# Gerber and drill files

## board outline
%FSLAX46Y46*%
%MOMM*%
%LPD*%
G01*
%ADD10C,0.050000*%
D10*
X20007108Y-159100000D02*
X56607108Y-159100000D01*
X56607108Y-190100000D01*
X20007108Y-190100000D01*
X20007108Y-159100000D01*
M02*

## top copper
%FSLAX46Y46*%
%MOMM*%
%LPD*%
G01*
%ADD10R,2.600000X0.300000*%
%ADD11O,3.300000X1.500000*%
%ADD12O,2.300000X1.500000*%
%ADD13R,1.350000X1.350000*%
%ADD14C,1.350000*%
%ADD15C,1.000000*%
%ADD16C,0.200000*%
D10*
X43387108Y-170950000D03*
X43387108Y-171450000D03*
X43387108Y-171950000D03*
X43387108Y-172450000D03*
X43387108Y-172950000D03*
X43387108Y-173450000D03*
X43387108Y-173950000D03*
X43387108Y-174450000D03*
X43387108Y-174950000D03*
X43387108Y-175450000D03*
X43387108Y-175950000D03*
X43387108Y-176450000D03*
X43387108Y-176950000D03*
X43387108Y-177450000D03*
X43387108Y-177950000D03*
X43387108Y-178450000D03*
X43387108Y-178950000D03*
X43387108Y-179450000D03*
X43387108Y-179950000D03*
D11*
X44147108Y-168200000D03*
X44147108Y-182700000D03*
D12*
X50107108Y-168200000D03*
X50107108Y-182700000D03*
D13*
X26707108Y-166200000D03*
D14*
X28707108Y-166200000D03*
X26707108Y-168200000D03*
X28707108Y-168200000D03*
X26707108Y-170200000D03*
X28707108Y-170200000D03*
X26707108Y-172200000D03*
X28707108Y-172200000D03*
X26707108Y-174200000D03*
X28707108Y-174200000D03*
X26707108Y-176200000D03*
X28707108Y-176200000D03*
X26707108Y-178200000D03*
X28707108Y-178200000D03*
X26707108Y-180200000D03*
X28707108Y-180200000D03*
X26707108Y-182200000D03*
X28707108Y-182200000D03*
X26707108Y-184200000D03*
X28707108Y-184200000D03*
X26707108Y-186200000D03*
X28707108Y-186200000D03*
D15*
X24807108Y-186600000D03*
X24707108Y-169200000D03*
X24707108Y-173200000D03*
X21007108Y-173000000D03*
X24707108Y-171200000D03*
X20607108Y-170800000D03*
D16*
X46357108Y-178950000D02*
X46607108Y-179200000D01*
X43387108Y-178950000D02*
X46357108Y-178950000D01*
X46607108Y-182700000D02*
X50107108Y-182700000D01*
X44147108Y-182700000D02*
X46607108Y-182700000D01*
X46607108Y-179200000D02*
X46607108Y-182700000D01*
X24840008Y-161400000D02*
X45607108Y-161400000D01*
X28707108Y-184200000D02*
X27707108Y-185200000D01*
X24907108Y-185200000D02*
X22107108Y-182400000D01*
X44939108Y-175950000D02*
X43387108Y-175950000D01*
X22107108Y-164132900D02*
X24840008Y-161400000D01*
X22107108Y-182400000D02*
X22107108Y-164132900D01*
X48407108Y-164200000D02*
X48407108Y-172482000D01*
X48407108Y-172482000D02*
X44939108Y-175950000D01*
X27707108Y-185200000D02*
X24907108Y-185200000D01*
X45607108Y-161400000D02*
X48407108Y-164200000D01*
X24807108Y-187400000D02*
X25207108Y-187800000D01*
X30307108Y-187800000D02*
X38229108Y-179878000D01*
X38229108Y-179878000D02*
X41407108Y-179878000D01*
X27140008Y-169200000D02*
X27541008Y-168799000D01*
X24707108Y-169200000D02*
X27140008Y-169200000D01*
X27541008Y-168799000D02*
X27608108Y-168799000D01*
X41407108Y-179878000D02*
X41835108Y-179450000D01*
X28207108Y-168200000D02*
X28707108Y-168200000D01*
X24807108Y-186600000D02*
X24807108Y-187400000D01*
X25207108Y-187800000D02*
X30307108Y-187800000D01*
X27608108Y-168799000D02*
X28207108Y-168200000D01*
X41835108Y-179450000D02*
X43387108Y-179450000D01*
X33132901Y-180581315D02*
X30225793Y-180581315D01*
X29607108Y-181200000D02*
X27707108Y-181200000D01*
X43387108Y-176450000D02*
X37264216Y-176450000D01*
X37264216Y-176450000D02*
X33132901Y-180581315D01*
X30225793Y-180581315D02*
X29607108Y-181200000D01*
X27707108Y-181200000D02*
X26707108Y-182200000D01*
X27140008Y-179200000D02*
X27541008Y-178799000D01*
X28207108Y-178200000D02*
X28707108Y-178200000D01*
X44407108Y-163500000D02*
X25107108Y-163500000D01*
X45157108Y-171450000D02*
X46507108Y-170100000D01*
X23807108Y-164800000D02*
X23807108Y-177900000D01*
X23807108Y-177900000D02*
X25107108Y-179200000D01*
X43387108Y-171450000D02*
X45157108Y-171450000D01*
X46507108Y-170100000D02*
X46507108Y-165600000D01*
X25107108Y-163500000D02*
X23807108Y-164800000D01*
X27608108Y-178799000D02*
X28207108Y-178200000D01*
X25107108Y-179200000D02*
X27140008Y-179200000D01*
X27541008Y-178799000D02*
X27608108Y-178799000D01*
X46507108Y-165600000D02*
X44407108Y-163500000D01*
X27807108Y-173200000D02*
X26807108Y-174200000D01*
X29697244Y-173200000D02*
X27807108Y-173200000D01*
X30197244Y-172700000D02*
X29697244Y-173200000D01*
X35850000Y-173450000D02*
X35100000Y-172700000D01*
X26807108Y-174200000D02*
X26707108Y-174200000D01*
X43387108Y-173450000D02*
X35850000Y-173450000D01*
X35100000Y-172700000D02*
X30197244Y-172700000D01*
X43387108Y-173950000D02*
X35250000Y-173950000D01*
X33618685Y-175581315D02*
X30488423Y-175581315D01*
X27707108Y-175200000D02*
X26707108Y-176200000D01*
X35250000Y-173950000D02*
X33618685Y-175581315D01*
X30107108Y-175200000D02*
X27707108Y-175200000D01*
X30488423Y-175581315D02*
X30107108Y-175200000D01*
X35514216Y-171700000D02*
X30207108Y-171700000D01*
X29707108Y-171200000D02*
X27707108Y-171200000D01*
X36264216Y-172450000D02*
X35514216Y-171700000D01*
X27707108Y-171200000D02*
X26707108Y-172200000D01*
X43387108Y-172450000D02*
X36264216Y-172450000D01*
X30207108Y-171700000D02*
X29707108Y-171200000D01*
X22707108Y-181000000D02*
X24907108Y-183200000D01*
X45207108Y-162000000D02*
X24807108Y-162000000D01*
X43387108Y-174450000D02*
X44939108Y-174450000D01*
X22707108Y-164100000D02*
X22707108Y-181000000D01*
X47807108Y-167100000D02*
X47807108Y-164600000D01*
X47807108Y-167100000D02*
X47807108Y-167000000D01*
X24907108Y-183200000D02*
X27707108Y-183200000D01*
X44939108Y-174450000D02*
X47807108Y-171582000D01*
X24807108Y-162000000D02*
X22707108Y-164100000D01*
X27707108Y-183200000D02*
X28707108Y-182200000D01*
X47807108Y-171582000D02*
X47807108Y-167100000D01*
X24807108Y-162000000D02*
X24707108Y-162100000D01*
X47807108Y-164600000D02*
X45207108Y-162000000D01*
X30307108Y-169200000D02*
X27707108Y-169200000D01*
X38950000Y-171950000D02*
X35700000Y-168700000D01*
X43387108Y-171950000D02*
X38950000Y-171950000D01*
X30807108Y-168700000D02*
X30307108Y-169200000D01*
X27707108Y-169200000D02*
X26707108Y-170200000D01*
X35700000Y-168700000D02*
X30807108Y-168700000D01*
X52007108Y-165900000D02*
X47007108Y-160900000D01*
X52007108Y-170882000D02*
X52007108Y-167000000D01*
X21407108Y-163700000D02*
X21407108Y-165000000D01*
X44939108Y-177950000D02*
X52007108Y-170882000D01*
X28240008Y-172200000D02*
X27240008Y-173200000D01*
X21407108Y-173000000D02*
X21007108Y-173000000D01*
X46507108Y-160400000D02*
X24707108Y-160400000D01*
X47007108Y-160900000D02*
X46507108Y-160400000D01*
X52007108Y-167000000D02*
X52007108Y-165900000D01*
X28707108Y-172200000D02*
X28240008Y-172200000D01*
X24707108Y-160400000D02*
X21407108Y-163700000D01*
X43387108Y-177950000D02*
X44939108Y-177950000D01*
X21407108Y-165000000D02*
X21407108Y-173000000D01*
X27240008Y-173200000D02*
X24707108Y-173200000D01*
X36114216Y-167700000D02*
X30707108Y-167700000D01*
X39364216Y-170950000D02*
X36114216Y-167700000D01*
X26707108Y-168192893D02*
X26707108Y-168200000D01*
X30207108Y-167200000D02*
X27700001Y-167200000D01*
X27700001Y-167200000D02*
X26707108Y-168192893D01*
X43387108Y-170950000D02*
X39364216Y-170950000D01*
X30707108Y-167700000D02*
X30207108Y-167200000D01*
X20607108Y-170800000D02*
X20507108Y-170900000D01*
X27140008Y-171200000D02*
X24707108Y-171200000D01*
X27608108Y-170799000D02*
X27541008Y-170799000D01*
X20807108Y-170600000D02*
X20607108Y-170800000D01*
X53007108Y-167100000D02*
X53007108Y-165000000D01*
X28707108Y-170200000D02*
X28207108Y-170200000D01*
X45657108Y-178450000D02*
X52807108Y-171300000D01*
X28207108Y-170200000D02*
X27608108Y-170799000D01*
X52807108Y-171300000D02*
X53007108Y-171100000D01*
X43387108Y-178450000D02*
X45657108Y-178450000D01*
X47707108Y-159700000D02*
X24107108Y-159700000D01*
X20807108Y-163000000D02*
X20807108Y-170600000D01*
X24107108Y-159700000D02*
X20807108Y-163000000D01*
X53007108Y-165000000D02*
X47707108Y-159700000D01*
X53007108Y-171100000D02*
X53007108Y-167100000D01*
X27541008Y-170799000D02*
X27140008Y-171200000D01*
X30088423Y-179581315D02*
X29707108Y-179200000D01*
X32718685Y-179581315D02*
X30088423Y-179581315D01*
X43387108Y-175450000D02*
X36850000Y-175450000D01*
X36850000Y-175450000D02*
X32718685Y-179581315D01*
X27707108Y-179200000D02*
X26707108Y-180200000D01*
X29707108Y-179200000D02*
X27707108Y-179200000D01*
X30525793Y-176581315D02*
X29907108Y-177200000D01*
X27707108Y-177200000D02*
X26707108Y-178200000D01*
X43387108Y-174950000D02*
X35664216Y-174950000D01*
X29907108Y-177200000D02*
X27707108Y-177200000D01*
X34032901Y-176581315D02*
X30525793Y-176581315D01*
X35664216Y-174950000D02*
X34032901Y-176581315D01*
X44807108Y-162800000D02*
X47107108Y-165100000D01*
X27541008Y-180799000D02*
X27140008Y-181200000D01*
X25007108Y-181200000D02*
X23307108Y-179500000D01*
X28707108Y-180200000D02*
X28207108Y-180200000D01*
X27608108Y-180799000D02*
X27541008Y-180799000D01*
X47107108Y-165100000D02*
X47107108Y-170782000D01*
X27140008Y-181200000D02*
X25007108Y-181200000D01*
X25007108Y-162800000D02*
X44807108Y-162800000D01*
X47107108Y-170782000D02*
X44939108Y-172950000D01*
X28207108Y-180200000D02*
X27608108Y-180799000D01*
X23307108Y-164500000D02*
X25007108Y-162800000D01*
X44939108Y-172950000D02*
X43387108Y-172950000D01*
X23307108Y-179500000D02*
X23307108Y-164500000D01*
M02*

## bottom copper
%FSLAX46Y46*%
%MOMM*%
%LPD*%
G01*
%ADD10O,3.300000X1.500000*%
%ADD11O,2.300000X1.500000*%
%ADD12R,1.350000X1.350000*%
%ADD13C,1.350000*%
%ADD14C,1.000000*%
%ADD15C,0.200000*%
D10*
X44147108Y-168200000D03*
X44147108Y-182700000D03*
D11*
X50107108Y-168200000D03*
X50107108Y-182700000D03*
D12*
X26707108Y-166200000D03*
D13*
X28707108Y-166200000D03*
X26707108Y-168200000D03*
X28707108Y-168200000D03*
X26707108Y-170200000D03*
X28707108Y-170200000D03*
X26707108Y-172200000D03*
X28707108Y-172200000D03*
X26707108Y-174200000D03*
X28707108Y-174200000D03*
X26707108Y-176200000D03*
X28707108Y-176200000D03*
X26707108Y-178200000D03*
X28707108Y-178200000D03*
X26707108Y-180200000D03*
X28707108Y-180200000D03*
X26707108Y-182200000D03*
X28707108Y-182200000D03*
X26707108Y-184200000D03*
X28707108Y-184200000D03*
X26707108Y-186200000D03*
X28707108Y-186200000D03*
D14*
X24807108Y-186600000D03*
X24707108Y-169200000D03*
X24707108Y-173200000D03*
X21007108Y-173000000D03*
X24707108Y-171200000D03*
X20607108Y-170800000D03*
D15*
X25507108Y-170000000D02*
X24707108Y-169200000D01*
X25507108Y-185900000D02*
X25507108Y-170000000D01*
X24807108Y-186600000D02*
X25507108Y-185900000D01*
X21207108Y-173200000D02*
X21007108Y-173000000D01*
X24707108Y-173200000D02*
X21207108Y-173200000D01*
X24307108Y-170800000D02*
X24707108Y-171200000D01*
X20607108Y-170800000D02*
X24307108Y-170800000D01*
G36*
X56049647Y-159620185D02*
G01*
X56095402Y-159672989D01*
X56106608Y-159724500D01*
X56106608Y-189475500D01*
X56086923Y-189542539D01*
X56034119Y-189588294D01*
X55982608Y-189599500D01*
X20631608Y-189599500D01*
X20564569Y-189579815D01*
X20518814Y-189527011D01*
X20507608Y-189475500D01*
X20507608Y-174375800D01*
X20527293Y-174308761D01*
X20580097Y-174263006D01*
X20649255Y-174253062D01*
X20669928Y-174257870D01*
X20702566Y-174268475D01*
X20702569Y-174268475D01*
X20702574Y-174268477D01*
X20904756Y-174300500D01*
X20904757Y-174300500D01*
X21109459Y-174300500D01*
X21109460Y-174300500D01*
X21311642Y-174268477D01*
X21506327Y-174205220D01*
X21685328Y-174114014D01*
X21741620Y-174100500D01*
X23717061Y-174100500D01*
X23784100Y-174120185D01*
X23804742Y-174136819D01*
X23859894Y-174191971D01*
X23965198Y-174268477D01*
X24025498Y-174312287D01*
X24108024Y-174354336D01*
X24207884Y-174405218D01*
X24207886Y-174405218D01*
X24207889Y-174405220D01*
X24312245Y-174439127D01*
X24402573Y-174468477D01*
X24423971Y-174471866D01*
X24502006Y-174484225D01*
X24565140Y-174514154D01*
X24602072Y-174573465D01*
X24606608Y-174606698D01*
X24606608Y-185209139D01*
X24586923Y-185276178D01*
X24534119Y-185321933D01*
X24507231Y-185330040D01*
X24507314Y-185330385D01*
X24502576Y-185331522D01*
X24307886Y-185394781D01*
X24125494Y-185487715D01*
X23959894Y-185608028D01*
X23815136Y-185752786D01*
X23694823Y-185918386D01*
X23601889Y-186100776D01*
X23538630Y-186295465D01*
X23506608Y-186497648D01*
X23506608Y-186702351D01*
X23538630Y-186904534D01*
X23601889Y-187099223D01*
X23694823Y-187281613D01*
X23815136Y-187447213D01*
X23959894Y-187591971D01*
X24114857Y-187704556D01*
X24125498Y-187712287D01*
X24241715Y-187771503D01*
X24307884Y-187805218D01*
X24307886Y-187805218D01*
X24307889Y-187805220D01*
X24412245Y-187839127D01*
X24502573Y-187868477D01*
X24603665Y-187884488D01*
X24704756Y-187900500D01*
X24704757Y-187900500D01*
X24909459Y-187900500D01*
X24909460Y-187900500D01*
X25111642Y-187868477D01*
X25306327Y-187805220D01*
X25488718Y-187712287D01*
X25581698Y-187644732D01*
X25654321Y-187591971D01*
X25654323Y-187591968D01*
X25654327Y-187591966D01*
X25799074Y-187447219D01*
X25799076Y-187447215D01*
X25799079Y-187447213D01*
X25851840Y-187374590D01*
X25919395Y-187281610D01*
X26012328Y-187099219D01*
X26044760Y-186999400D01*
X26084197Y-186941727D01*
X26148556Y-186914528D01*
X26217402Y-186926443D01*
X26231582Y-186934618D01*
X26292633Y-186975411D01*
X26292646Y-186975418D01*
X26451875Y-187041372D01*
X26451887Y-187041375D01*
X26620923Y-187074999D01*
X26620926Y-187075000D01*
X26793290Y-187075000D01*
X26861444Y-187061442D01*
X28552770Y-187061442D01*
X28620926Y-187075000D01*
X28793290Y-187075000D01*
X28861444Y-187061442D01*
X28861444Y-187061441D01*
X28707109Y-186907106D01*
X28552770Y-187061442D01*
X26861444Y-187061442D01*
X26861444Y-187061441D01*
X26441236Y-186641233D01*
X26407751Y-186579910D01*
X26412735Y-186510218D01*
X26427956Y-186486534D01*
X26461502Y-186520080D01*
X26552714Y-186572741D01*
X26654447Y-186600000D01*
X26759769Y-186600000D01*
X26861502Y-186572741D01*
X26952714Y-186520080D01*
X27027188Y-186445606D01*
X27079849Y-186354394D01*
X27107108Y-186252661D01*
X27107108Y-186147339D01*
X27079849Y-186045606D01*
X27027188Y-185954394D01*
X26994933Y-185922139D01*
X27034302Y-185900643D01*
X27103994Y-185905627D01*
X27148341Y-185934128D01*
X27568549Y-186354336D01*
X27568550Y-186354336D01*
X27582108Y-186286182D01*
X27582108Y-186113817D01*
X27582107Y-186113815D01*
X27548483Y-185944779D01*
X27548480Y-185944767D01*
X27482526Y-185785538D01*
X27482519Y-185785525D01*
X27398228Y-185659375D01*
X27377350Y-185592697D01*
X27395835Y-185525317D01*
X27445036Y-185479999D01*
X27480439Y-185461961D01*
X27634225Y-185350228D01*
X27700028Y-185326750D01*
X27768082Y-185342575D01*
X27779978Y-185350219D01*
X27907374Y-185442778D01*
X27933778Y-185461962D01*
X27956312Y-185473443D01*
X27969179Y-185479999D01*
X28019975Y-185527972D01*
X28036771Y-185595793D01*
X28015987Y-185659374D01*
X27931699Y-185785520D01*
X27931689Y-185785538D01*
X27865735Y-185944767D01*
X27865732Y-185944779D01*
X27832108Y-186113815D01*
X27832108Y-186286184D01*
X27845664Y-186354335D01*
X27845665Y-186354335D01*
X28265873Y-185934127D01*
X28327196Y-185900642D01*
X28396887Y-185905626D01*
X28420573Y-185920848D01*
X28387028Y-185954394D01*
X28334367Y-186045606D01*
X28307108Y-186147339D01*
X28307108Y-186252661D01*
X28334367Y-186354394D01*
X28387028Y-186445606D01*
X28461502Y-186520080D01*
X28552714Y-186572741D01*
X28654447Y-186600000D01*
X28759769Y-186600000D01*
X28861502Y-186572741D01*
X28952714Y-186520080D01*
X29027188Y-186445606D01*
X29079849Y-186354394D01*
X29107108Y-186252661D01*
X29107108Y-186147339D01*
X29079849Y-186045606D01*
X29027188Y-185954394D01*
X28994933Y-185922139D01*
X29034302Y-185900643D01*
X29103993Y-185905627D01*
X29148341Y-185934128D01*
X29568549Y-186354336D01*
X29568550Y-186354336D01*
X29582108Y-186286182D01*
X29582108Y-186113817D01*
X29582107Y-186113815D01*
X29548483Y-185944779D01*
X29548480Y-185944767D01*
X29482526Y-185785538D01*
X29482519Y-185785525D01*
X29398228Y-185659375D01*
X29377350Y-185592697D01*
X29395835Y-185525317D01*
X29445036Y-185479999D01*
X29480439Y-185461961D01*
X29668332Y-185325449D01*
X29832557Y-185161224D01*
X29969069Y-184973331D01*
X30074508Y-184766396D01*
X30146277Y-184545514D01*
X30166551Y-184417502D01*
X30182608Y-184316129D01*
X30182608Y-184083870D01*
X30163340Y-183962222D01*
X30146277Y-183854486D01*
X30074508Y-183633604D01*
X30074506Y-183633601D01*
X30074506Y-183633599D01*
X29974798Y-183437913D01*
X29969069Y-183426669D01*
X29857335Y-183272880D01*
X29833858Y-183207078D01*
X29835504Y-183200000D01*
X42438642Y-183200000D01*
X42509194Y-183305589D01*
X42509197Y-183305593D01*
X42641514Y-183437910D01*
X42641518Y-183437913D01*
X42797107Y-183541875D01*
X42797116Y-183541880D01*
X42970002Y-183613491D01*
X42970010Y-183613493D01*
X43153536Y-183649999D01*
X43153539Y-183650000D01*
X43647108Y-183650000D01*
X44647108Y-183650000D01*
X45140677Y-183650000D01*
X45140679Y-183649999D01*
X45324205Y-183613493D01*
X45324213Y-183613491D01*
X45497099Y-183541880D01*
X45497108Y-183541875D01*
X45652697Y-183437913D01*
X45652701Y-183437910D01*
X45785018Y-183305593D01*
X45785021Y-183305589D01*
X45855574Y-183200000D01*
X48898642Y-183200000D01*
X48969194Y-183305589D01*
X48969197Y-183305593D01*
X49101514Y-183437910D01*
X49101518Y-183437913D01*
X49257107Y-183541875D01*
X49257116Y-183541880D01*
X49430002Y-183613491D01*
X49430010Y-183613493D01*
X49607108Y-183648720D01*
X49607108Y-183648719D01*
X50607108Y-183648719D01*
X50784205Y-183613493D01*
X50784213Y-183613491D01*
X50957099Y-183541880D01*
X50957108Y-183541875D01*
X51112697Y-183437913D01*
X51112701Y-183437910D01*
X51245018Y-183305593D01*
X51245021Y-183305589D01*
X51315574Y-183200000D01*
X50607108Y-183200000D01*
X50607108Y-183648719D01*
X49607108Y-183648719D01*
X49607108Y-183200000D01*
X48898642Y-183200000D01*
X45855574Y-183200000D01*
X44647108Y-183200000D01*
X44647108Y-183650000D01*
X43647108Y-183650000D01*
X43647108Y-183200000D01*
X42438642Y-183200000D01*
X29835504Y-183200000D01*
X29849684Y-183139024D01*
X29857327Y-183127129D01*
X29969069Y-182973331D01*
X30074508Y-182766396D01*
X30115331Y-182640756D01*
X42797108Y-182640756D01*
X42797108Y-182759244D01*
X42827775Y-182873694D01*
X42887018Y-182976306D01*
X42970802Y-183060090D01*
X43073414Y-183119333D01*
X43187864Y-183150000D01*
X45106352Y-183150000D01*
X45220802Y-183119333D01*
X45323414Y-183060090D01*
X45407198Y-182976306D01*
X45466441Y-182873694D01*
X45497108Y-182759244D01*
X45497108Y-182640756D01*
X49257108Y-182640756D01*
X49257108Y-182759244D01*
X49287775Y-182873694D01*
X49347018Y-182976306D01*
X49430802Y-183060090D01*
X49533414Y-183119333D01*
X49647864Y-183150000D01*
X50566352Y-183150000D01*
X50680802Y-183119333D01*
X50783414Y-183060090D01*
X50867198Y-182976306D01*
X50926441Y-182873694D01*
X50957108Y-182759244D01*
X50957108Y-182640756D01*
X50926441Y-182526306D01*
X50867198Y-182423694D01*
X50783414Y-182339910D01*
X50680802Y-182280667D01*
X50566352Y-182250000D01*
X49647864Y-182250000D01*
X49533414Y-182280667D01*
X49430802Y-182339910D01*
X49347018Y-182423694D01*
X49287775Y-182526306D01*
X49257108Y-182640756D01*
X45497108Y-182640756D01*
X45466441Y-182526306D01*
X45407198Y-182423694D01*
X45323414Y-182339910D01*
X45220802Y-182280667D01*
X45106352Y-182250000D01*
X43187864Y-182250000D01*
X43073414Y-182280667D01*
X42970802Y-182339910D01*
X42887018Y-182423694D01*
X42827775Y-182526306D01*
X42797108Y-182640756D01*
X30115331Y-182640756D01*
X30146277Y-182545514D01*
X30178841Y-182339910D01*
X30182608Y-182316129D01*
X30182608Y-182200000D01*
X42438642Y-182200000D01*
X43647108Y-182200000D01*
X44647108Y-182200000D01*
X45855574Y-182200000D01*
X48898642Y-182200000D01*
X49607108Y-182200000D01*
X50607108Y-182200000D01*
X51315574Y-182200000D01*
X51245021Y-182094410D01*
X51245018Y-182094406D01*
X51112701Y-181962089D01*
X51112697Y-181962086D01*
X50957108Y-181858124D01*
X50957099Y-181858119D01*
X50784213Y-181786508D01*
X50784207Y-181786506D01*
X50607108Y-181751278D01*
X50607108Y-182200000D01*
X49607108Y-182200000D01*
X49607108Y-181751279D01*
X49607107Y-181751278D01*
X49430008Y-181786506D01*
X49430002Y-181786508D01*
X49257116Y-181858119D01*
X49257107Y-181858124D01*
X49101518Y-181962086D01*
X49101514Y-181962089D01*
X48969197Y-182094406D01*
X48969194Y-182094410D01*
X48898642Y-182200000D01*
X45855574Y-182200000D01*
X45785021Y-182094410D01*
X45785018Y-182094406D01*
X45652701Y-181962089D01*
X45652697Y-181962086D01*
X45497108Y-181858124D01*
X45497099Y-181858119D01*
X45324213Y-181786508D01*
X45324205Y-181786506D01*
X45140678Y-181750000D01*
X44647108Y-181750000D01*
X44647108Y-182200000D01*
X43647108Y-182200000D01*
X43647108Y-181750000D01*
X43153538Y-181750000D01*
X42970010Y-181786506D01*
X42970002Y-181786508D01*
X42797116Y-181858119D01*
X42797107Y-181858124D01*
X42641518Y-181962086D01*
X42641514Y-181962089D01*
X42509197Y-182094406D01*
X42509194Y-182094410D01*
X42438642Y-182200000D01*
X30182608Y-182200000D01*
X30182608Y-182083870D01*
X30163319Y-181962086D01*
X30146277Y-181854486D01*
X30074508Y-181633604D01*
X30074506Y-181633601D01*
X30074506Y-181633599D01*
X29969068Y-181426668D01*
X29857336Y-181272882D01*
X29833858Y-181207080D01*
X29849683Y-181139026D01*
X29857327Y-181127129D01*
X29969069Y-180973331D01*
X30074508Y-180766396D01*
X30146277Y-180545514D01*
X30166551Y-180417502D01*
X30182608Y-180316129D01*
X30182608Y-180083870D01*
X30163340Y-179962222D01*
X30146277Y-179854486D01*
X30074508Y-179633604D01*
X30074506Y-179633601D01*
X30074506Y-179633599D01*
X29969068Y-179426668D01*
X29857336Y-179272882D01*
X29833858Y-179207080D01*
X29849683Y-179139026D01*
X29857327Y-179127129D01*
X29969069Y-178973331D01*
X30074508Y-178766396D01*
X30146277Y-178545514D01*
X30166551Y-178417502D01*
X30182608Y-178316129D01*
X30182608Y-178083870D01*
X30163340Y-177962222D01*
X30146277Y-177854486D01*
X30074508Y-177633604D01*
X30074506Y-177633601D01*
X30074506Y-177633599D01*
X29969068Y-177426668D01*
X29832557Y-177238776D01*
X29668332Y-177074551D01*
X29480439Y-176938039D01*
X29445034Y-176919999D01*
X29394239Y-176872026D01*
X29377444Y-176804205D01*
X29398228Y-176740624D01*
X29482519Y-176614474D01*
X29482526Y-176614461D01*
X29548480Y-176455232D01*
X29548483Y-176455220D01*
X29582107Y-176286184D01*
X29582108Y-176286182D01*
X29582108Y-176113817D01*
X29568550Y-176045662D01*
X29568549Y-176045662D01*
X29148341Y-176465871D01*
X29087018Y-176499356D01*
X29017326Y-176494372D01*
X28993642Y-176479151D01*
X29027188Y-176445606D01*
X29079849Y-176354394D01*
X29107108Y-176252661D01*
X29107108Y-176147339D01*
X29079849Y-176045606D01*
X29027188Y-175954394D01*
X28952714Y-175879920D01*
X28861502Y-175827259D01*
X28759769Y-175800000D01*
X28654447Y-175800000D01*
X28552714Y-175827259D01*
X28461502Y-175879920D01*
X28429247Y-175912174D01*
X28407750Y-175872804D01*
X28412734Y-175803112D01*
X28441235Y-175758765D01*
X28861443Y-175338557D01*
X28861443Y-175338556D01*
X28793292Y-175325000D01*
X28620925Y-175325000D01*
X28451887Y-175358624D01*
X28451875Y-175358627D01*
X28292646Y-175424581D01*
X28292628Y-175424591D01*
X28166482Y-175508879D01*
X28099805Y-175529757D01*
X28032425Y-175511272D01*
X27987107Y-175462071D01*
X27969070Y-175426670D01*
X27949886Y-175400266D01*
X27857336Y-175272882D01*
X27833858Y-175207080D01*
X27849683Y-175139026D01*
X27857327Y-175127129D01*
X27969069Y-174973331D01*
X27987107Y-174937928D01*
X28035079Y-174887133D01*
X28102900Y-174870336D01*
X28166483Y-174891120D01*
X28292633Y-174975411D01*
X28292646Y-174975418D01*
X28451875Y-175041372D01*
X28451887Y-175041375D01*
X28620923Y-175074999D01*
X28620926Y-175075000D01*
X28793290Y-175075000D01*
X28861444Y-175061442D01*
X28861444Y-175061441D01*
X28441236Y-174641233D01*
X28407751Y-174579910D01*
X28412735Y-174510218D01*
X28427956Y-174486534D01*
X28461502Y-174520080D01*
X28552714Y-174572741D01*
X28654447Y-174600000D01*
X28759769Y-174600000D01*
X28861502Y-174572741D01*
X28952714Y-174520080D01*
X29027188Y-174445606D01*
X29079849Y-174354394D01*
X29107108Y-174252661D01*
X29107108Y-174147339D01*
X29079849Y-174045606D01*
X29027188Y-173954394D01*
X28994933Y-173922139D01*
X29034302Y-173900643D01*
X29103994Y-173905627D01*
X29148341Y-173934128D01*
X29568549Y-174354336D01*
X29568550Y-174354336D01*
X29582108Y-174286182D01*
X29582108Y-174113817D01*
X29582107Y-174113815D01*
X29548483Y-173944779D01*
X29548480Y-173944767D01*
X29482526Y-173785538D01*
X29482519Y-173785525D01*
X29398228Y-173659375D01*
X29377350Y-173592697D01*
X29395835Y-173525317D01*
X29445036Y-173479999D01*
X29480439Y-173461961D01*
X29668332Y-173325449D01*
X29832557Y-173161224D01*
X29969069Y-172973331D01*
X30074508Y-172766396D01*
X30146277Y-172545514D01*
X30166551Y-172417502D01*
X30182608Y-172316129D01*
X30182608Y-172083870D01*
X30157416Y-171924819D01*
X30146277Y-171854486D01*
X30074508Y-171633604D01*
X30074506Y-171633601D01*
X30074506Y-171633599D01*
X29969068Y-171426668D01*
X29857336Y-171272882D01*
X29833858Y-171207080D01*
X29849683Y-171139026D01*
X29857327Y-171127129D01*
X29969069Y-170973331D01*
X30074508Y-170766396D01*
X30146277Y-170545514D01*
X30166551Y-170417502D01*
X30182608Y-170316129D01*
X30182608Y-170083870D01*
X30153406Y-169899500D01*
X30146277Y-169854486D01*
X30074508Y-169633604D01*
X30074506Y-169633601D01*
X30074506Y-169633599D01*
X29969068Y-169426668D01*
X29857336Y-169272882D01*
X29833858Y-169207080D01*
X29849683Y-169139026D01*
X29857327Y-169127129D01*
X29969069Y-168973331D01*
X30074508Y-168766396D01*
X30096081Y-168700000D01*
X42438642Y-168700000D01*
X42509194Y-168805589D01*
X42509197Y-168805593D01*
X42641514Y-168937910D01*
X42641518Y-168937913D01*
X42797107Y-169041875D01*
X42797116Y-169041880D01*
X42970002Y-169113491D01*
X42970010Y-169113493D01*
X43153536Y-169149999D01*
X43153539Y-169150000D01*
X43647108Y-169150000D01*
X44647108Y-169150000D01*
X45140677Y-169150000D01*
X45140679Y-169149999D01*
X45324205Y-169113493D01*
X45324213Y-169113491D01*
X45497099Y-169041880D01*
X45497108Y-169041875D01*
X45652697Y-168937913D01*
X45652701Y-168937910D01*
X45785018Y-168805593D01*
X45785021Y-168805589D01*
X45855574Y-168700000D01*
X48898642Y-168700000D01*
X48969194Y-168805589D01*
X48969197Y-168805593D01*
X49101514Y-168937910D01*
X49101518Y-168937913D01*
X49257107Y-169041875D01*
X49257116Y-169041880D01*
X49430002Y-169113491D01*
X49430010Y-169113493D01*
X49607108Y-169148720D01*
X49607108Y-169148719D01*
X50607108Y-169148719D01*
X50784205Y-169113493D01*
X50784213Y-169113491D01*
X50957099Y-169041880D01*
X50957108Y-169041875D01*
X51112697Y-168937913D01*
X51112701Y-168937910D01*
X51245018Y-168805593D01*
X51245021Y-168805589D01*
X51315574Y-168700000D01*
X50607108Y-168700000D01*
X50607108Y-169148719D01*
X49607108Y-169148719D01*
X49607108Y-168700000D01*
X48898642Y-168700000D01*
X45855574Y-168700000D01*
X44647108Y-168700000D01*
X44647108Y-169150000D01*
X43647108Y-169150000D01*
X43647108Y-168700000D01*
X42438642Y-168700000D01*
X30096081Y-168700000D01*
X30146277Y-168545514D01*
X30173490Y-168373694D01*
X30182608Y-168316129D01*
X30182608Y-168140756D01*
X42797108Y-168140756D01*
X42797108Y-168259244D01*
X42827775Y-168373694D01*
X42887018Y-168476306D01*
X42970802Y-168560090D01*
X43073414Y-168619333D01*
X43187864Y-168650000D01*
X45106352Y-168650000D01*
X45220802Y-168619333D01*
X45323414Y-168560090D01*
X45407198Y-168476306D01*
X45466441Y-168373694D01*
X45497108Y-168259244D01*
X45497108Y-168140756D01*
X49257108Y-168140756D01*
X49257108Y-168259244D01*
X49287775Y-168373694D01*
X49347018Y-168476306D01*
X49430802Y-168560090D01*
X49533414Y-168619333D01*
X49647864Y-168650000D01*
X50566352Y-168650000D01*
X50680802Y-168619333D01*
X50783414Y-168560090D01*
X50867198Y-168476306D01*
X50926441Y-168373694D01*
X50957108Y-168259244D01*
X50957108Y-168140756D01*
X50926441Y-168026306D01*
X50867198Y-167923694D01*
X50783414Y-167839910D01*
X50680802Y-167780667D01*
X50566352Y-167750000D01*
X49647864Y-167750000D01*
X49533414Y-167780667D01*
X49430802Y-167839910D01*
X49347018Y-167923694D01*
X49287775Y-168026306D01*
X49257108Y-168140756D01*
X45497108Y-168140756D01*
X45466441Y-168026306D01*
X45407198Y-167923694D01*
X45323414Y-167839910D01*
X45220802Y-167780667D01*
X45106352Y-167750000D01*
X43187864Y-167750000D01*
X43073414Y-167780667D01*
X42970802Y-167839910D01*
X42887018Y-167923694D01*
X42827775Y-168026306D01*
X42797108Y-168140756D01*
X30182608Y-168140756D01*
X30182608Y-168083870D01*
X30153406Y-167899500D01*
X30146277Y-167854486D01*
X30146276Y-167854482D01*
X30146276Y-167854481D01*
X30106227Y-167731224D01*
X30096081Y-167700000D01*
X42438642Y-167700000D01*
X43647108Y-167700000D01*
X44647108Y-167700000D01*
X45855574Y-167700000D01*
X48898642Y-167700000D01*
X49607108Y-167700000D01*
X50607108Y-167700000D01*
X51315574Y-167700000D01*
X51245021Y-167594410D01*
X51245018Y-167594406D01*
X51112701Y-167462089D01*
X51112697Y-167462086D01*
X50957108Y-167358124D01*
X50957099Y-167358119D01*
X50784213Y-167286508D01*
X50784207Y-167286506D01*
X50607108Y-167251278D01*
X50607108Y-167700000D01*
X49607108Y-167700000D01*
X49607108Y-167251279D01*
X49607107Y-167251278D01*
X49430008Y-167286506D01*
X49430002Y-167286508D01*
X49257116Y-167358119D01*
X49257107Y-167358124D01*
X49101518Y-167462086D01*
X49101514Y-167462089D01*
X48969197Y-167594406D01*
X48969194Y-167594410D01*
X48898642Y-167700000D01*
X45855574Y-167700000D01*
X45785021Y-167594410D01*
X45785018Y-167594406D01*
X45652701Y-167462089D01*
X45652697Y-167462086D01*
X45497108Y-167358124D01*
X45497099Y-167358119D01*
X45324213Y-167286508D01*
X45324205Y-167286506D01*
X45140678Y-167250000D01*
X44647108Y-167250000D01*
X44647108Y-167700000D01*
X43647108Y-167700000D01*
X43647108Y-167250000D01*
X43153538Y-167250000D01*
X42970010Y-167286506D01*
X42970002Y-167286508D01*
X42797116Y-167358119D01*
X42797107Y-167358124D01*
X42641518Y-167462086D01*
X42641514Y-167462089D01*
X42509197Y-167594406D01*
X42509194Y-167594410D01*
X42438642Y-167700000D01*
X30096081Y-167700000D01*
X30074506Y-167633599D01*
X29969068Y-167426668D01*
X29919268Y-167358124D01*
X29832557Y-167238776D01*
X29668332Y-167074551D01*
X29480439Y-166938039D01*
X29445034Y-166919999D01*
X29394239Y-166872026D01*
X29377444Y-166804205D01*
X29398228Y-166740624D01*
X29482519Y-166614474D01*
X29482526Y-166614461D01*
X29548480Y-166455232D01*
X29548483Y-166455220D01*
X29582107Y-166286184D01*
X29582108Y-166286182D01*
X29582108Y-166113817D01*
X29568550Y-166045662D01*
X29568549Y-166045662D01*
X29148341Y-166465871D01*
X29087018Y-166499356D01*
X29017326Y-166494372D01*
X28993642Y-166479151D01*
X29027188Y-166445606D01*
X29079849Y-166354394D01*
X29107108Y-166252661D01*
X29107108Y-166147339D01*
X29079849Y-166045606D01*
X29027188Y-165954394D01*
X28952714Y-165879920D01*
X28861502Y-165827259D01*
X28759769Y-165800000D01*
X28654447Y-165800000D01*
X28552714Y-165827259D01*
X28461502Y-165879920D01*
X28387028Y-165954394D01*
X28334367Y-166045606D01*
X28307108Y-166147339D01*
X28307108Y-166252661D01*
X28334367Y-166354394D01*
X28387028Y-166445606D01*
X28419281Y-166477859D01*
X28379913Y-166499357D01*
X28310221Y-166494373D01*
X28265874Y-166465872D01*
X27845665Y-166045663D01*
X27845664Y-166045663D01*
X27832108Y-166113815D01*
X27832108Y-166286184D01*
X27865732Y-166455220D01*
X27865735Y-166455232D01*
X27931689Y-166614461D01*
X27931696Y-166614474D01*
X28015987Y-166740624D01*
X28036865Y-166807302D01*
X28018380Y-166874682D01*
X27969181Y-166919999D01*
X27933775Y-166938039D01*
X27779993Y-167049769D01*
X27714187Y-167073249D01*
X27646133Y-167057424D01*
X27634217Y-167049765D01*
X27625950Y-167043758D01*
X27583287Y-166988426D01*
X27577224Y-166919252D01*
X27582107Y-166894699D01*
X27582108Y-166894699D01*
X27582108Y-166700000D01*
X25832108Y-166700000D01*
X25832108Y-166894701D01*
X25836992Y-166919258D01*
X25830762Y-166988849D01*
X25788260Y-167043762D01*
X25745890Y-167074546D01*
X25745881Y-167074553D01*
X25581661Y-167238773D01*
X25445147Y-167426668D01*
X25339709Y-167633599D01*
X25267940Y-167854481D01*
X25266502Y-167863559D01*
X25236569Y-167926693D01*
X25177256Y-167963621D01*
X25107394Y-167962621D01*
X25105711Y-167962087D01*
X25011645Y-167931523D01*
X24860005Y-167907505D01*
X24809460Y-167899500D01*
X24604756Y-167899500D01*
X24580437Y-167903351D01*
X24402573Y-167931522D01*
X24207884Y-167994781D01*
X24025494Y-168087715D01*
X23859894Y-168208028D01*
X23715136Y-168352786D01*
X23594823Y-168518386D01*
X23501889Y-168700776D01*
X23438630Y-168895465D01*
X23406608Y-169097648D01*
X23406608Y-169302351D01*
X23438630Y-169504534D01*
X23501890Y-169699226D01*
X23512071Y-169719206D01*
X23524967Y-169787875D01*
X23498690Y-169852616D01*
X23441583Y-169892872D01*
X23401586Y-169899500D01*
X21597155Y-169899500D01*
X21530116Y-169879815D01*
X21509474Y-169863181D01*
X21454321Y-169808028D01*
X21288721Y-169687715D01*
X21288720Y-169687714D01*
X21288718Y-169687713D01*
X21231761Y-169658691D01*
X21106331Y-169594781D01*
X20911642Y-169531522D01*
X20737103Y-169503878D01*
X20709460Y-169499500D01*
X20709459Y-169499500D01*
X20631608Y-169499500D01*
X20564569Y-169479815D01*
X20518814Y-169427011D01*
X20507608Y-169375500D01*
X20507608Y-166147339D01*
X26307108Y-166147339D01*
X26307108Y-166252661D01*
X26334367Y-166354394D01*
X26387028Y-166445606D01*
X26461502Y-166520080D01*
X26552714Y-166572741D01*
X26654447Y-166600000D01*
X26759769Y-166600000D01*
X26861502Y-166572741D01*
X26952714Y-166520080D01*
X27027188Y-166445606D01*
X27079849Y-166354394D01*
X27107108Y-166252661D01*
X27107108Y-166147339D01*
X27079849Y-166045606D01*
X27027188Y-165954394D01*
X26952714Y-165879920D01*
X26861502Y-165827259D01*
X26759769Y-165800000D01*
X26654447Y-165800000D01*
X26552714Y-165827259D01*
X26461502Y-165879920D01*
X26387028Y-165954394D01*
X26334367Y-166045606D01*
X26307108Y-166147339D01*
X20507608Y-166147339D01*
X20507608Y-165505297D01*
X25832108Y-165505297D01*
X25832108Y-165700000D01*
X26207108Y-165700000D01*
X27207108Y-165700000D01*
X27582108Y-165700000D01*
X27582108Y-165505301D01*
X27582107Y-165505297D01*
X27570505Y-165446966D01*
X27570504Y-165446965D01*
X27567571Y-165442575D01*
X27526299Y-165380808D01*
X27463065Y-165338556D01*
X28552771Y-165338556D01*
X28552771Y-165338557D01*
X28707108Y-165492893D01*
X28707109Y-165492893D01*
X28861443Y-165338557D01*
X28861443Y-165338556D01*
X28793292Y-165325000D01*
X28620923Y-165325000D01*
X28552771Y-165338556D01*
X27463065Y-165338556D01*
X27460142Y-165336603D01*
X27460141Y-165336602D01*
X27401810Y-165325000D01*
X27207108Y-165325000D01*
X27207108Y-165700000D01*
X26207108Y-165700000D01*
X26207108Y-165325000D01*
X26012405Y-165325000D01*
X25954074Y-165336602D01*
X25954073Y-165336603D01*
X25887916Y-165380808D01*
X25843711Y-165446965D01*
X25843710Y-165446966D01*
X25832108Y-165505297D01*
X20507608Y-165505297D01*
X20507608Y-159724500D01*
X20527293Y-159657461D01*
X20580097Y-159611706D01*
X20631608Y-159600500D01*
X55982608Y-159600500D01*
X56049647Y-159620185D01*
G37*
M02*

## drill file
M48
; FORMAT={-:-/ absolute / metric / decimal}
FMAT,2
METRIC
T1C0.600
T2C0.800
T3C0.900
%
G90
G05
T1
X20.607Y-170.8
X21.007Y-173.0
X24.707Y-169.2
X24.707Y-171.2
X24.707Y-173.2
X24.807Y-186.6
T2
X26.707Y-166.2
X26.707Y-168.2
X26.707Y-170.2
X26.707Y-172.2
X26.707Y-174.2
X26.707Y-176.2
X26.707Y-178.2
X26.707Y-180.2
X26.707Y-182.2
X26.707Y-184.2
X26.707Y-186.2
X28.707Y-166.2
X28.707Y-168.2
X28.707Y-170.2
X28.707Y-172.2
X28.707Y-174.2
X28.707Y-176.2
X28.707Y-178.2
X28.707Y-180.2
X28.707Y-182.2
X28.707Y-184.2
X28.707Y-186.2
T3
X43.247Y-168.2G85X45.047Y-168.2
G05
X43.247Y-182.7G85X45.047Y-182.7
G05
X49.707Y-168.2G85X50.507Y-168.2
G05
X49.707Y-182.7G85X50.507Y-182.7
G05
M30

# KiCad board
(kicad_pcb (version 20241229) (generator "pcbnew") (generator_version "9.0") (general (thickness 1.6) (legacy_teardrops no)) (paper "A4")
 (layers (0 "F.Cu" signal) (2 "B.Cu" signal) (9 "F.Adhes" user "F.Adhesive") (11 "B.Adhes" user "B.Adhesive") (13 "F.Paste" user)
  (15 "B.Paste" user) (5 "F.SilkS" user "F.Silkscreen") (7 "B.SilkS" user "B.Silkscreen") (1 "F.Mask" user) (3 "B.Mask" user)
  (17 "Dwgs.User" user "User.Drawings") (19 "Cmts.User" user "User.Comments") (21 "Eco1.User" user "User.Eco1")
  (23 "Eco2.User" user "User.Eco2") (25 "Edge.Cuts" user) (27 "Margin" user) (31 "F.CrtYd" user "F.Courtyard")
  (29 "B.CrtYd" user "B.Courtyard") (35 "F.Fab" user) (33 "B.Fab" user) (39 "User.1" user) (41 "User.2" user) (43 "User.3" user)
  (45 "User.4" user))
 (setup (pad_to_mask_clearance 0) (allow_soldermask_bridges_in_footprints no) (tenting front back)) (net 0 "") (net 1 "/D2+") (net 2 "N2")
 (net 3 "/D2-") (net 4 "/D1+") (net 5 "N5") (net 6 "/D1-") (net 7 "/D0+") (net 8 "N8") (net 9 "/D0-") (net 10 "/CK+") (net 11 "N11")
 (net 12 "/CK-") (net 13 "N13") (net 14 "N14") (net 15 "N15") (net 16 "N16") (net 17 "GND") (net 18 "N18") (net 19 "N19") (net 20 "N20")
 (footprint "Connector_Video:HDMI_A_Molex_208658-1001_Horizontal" (layer "F.Cu") (at 46.672108 175.45)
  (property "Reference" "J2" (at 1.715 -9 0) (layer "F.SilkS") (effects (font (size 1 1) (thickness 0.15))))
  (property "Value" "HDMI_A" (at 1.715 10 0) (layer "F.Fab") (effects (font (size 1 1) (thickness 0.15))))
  (pad "1" smd rect (at -3.285 -4.5) (size 2.6 0.3) (layers "F.Cu" "F.Mask" "F.Paste") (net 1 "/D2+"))
  (pad "2" smd rect (at -3.285 -4) (size 2.6 0.3) (layers "F.Cu" "F.Mask" "F.Paste") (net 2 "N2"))
  (pad "3" smd rect (at -3.285 -3.5) (size 2.6 0.3) (layers "F.Cu" "F.Mask" "F.Paste") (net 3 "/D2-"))
  (pad "4" smd rect (at -3.285 -3) (size 2.6 0.3) (layers "F.Cu" "F.Mask" "F.Paste") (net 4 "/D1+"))
  (pad "5" smd rect (at -3.285 -2.5) (size 2.6 0.3) (layers "F.Cu" "F.Mask" "F.Paste") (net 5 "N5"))
  (pad "6" smd rect (at -3.285 -2) (size 2.6 0.3) (layers "F.Cu" "F.Mask" "F.Paste") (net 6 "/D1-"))
  (pad "7" smd rect (at -3.285 -1.5) (size 2.6 0.3) (layers "F.Cu" "F.Mask" "F.Paste") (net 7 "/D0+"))
  (pad "8" smd rect (at -3.285 -1) (size 2.6 0.3) (layers "F.Cu" "F.Mask" "F.Paste") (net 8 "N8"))
  (pad "9" smd rect (at -3.285 -0.5) (size 2.6 0.3) (layers "F.Cu" "F.Mask" "F.Paste") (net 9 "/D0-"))
  (pad "10" smd rect (at -3.285 0) (size 2.6 0.3) (layers "F.Cu" "F.Mask" "F.Paste") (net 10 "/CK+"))
  (pad "11" smd rect (at -3.285 0.5) (size 2.6 0.3) (layers "F.Cu" "F.Mask" "F.Paste") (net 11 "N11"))
  (pad "12" smd rect (at -3.285 1) (size 2.6 0.3) (layers "F.Cu" "F.Mask" "F.Paste") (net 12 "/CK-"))
  (pad "13" smd rect (at -3.285 1.5) (size 2.6 0.3) (layers "F.Cu" "F.Mask" "F.Paste") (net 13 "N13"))
  (pad "14" smd rect (at -3.285 2) (size 2.6 0.3) (layers "F.Cu" "F.Mask" "F.Paste") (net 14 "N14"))
  (pad "15" smd rect (at -3.285 2.5) (size 2.6 0.3) (layers "F.Cu" "F.Mask" "F.Paste") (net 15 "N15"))
  (pad "16" smd rect (at -3.285 3) (size 2.6 0.3) (layers "F.Cu" "F.Mask" "F.Paste") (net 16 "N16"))
  (pad "17" smd rect (at -3.285 3.5) (size 2.6 0.3) (layers "F.Cu" "F.Mask" "F.Paste") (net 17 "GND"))
  (pad "18" smd rect (at -3.285 4) (size 2.6 0.3) (layers "F.Cu" "F.Mask" "F.Paste") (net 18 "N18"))
  (pad "19" smd rect (at -3.285 4.5) (size 2.6 0.3) (layers "F.Cu" "F.Mask" "F.Paste") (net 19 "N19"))
  (pad "SH" thru_hole oval (at -2.525 -7.25) (size 3.3 1.5) (drill oval 2.7 0.9) (layers "*.Cu" "*.Mask") (remove_unused_layers no)
   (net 17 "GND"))
  (pad "SH" thru_hole oval (at -2.525 7.25) (size 3.3 1.5) (drill oval 2.7 0.9) (layers "*.Cu" "*.Mask") (remove_unused_layers no)
   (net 17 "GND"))
  (pad "SH" thru_hole oval (at 3.435 -7.25) (size 2.3 1.5) (drill oval 1.7 0.9) (layers "*.Cu" "*.Mask") (remove_unused_layers no)
   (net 17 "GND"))
  (pad "SH" thru_hole oval (at 3.435 7.25) (size 2.3 1.5) (drill oval 1.7 0.9) (layers "*.Cu" "*.Mask") (remove_unused_layers no)
   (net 17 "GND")))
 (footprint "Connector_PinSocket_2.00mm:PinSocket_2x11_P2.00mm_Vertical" (layer "B.Cu") (at 26.707108 166.2 180)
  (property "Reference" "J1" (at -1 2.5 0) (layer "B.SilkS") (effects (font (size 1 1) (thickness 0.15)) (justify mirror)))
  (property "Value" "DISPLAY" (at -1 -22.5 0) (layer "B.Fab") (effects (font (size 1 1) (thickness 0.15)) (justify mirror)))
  (pad "1" thru_hole rect (at 0 0 180) (size 1.35 1.35) (drill 0.8) (layers "*.Cu" "*.Mask") (remove_unused_layers no) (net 17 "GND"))
  (pad "2" thru_hole circle (at -2 0 180) (size 1.35 1.35) (drill 0.8) (layers "*.Cu" "*.Mask") (remove_unused_layers no) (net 17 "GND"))
  (pad "3" thru_hole circle (at 0 -2 180) (size 1.35 1.35) (drill 0.8) (layers "*.Cu" "*.Mask") (remove_unused_layers no) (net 1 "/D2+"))
  (pad "4" thru_hole circle (at -2 -2 180) (size 1.35 1.35) (drill 0.8) (layers "*.Cu" "*.Mask") (remove_unused_layers no) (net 18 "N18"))
  (pad "5" thru_hole circle (at 0 -4 180) (size 1.35 1.35) (drill 0.8) (layers "*.Cu" "*.Mask") (remove_unused_layers no) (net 3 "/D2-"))
  (pad "6" thru_hole circle (at -2 -4 180) (size 1.35 1.35) (drill 0.8) (layers "*.Cu" "*.Mask") (remove_unused_layers no) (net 16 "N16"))
  (pad "7" thru_hole circle (at 0 -6 180) (size 1.35 1.35) (drill 0.8) (layers "*.Cu" "*.Mask") (remove_unused_layers no) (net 4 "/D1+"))
  (pad "8" thru_hole circle (at -2 -6 180) (size 1.35 1.35) (drill 0.8) (layers "*.Cu" "*.Mask") (remove_unused_layers no) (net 15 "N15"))
  (pad "9" thru_hole circle (at 0 -8 180) (size 1.35 1.35) (drill 0.8) (layers "*.Cu" "*.Mask") (remove_unused_layers no) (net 6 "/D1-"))
  (pad "10" thru_hole circle (at -2 -8 180) (size 1.35 1.35) (drill 0.8) (layers "*.Cu" "*.Mask") (remove_unused_layers no) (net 17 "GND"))
  (pad "11" thru_hole circle (at 0 -10 180) (size 1.35 1.35) (drill 0.8) (layers "*.Cu" "*.Mask") (remove_unused_layers no) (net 7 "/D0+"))
  (pad "12" thru_hole circle (at -2 -10 180) (size 1.35 1.35) (drill 0.8) (layers "*.Cu" "*.Mask") (remove_unused_layers no) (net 17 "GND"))
  (pad "13" thru_hole circle (at 0 -12 180) (size 1.35 1.35) (drill 0.8) (layers "*.Cu" "*.Mask") (remove_unused_layers no) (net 9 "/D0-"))
  (pad "14" thru_hole circle (at -2 -12 180) (size 1.35 1.35) (drill 0.8) (layers "*.Cu" "*.Mask") (remove_unused_layers no) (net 2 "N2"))
  (pad "15" thru_hole circle (at 0 -14 180) (size 1.35 1.35) (drill 0.8) (layers "*.Cu" "*.Mask") (remove_unused_layers no) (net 10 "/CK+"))
  (pad "16" thru_hole circle (at -2 -14 180) (size 1.35 1.35) (drill 0.8) (layers "*.Cu" "*.Mask") (remove_unused_layers no) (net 5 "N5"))
  (pad "17" thru_hole circle (at 0 -16 180) (size 1.35 1.35) (drill 0.8) (layers "*.Cu" "*.Mask") (remove_unused_layers no) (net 12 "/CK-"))
  (pad "18" thru_hole circle (at -2 -16 180) (size 1.35 1.35) (drill 0.8) (layers "*.Cu" "*.Mask") (remove_unused_layers no) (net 8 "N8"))
  (pad "19" thru_hole circle (at 0 -18 180) (size 1.35 1.35) (drill 0.8) (layers "*.Cu" "*.Mask") (remove_unused_layers no) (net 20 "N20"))
  (pad "20" thru_hole circle (at -2 -18 180) (size 1.35 1.35) (drill 0.8) (layers "*.Cu" "*.Mask") (remove_unused_layers no) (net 11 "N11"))
  (pad "21" thru_hole circle (at 0 -20 180) (size 1.35 1.35) (drill 0.8) (layers "*.Cu" "*.Mask") (remove_unused_layers no) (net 17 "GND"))
  (pad "22" thru_hole circle (at -2 -20 180) (size 1.35 1.35) (drill 0.8) (layers "*.Cu" "*.Mask") (remove_unused_layers no) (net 17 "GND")))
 (gr_rect (start 20.007108 159.1) (end 56.607108 190.1) (stroke (width 0.05) (type default)) (fill no) (layer "Edge.Cuts"))
 (segment (start 46.357108 178.95) (end 46.607108 179.2) (width 0.2) (layer "F.Cu") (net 17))
 (segment (start 43.387108 178.95) (end 46.357108 178.95) (width 0.2) (layer "F.Cu") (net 17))
 (segment (start 46.607108 182.7) (end 50.107108 182.7) (width 0.2) (layer "F.Cu") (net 17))
 (segment (start 44.147108 182.7) (end 46.607108 182.7) (width 0.2) (layer "F.Cu") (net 17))
 (segment (start 46.607108 179.2) (end 46.607108 182.7) (width 0.2) (layer "F.Cu") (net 17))
 (segment (start 24.840008 161.4) (end 45.607108 161.4) (width 0.2) (layer "F.Cu") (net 11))
 (segment (start 28.707108 184.2) (end 27.707108 185.2) (width 0.2) (layer "F.Cu") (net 11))
 (segment (start 24.907108 185.2) (end 22.107108 182.4) (width 0.2) (layer "F.Cu") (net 11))
 (segment (start 44.939108 175.95) (end 43.387108 175.95) (width 0.2) (layer "F.Cu") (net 11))
 (segment (start 22.107108 164.1329) (end 24.840008 161.4) (width 0.2) (layer "F.Cu") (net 11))
 (segment (start 22.107108 182.4) (end 22.107108 164.1329) (width 0.2) (layer "F.Cu") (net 11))
 (segment (start 48.407108 164.2) (end 48.407108 172.482) (width 0.2) (layer "F.Cu") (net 11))
 (segment (start 48.407108 172.482) (end 44.939108 175.95) (width 0.2) (layer "F.Cu") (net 11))
 (segment (start 27.707108 185.2) (end 24.907108 185.2) (width 0.2) (layer "F.Cu") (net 11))
 (segment (start 45.607108 161.4) (end 48.407108 164.2) (width 0.2) (layer "F.Cu") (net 11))
 (segment (start 24.807108 187.4) (end 25.207108 187.8) (width 0.2) (layer "F.Cu") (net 18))
 (segment (start 30.307108 187.8) (end 38.229108 179.878) (width 0.2) (layer "F.Cu") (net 18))
 (segment (start 38.229108 179.878) (end 41.407108 179.878) (width 0.2) (layer "F.Cu") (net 18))
 (segment (start 27.140008 169.2) (end 27.541008 168.799) (width 0.2) (layer "F.Cu") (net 18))
 (segment (start 24.707108 169.2) (end 27.140008 169.2) (width 0.2) (layer "F.Cu") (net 18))
 (segment (start 27.541008 168.799) (end 27.608108 168.799) (width 0.2) (layer "F.Cu") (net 18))
 (segment (start 41.407108 179.878) (end 41.835108 179.45) (width 0.2) (layer "F.Cu") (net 18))
 (segment (start 28.207108 168.2) (end 28.707108 168.2) (width 0.2) (layer "F.Cu") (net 18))
 (segment (start 24.807108 186.6) (end 24.807108 187.4) (width 0.2) (layer "F.Cu") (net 18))
 (segment (start 25.207108 187.8) (end 30.307108 187.8) (width 0.2) (layer "F.Cu") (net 18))
 (segment (start 27.608108 168.799) (end 28.207108 168.2) (width 0.2) (layer "F.Cu") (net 18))
 (segment (start 41.835108 179.45) (end 43.387108 179.45) (width 0.2) (layer "F.Cu") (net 18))
 (via (at 24.807108 186.6) (size 1) (drill 0.6) (layers "F.Cu" "B.Cu") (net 18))
 (via (at 24.707108 169.2) (size 1) (drill 0.6) (layers "F.Cu" "B.Cu") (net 18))
 (segment (start 25.507108 170) (end 24.707108 169.2) (width 0.2) (layer "B.Cu") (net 18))
 (segment (start 25.507108 185.9) (end 25.507108 170) (width 0.2) (layer "B.Cu") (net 18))
 (segment (start 24.807108 186.6) (end 25.507108 185.9) (width 0.2) (layer "B.Cu") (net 18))
 (segment (start 33.132901 180.581315) (end 30.225793 180.581315) (width 0.2) (layer "F.Cu") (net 12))
 (segment (start 29.607108 181.2) (end 27.707108 181.2) (width 0.2) (layer "F.Cu") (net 12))
 (segment (start 43.387108 176.45) (end 37.264216 176.45) (width 0.2) (layer "F.Cu") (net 12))
 (segment (start 37.264216 176.45) (end 33.132901 180.581315) (width 0.2) (layer "F.Cu") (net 12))
 (segment (start 30.225793 180.581315) (end 29.607108 181.2) (width 0.2) (layer "F.Cu") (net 12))
 (segment (start 27.707108 181.2) (end 26.707108 182.2) (width 0.2) (layer "F.Cu") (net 12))
 (segment (start 27.140008 179.2) (end 27.541008 178.799) (width 0.2) (layer "F.Cu") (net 2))
 (segment (start 28.207108 178.2) (end 28.707108 178.2) (width 0.2) (layer "F.Cu") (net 2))
 (segment (start 44.407108 163.5) (end 25.107108 163.5) (width 0.2) (layer "F.Cu") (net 2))
 (segment (start 45.157108 171.45) (end 46.507108 170.1) (width 0.2) (layer "F.Cu") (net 2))
 (segment (start 23.807108 164.8) (end 23.807108 177.9) (width 0.2) (layer "F.Cu") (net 2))
 (segment (start 23.807108 177.9) (end 25.107108 179.2) (width 0.2) (layer "F.Cu") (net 2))
 (segment (start 43.387108 171.45) (end 45.157108 171.45) (width 0.2) (layer "F.Cu") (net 2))
 (segment (start 46.507108 170.1) (end 46.507108 165.6) (width 0.2) (layer "F.Cu") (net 2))
 (segment (start 25.107108 163.5) (end 23.807108 164.8) (width 0.2) (layer "F.Cu") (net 2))
 (segment (start 27.608108 178.799) (end 28.207108 178.2) (width 0.2) (layer "F.Cu") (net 2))
 (segment (start 25.107108 179.2) (end 27.140008 179.2) (width 0.2) (layer "F.Cu") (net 2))
 (segment (start 27.541008 178.799) (end 27.608108 178.799) (width 0.2) (layer "F.Cu") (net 2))
 (segment (start 46.507108 165.6) (end 44.407108 163.5) (width 0.2) (layer "F.Cu") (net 2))
 (segment (start 27.807108 173.2) (end 26.807108 174.2) (width 0.2) (layer "F.Cu") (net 6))
 (segment (start 29.697244 173.2) (end 27.807108 173.2) (width 0.2) (layer "F.Cu") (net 6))
 (segment (start 30.197244 172.7) (end 29.697244 173.2) (width 0.2) (layer "F.Cu") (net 6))
 (segment (start 35.85 173.45) (end 35.1 172.7) (width 0.2) (layer "F.Cu") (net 6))
 (segment (start 26.807108 174.2) (end 26.707108 174.2) (width 0.2) (layer "F.Cu") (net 6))
 (segment (start 43.387108 173.45) (end 35.85 173.45) (width 0.2) (layer "F.Cu") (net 6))
 (segment (start 35.1 172.7) (end 30.197244 172.7) (width 0.2) (layer "F.Cu") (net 6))
 (segment (start 43.387108 173.95) (end 35.25 173.95) (width 0.2) (layer "F.Cu") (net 7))
 (segment (start 33.618685 175.581315) (end 30.488423 175.581315) (width 0.2) (layer "F.Cu") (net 7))
 (segment (start 27.707108 175.2) (end 26.707108 176.2) (width 0.2) (layer "F.Cu") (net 7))
 (segment (start 35.25 173.95) (end 33.618685 175.581315) (width 0.2) (layer "F.Cu") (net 7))
 (segment (start 30.107108 175.2) (end 27.707108 175.2) (width 0.2) (layer "F.Cu") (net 7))
 (segment (start 30.488423 175.581315) (end 30.107108 175.2) (width 0.2) (layer "F.Cu") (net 7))
 (segment (start 35.514216 171.7) (end 30.207108 171.7) (width 0.2) (layer "F.Cu") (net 4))
 (segment (start 29.707108 171.2) (end 27.707108 171.2) (width 0.2) (layer "F.Cu") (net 4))
 (segment (start 36.264216 172.45) (end 35.514216 171.7) (width 0.2) (layer "F.Cu") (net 4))
 (segment (start 27.707108 171.2) (end 26.707108 172.2) (width 0.2) (layer "F.Cu") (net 4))
 (segment (start 43.387108 172.45) (end 36.264216 172.45) (width 0.2) (layer "F.Cu") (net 4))
 (segment (start 30.207108 171.7) (end 29.707108 171.2) (width 0.2) (layer "F.Cu") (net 4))
 (segment (start 22.707108 181) (end 24.907108 183.2) (width 0.2) (layer "F.Cu") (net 8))
 (segment (start 45.207108 162) (end 24.807108 162) (width 0.2) (layer "F.Cu") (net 8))
 (segment (start 43.387108 174.45) (end 44.939108 174.45) (width 0.2) (layer "F.Cu") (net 8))
 (segment (start 22.707108 164.1) (end 22.707108 181) (width 0.2) (layer "F.Cu") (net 8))
 (segment (start 47.807108 167.1) (end 47.807108 164.6) (width 0.2) (layer "F.Cu") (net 8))
 (segment (start 47.807108 167.1) (end 47.807108 167) (width 0.2) (layer "F.Cu") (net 8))
 (segment (start 24.907108 183.2) (end 27.707108 183.2) (width 0.2) (layer "F.Cu") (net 8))
 (segment (start 44.939108 174.45) (end 47.807108 171.582) (width 0.2) (layer "F.Cu") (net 8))
 (segment (start 24.807108 162) (end 22.707108 164.1) (width 0.2) (layer "F.Cu") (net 8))
 (segment (start 27.707108 183.2) (end 28.707108 182.2) (width 0.2) (layer "F.Cu") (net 8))
 (segment (start 47.807108 171.582) (end 47.807108 167.1) (width 0.2) (layer "F.Cu") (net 8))
 (segment (start 24.807108 162) (end 24.707108 162.1) (width 0.2) (layer "F.Cu") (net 8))
 (segment (start 47.807108 164.6) (end 45.207108 162) (width 0.2) (layer "F.Cu") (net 8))
 (segment (start 30.307108 169.2) (end 27.707108 169.2) (width 0.2) (layer "F.Cu") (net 3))
 (segment (start 38.95 171.95) (end 35.7 168.7) (width 0.2) (layer "F.Cu") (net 3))
 (segment (start 43.387108 171.95) (end 38.95 171.95) (width 0.2) (layer "F.Cu") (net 3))
 (segment (start 30.807108 168.7) (end 30.307108 169.2) (width 0.2) (layer "F.Cu") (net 3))
 (segment (start 27.707108 169.2) (end 26.707108 170.2) (width 0.2) (layer "F.Cu") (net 3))
 (segment (start 35.7 168.7) (end 30.807108 168.7) (width 0.2) (layer "F.Cu") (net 3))
 (segment (start 52.007108 165.9) (end 47.007108 160.9) (width 0.2) (layer "F.Cu") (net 15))
 (segment (start 52.007108 170.882) (end 52.007108 167) (width 0.2) (layer "F.Cu") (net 15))
 (segment (start 21.407108 163.7) (end 21.407108 165) (width 0.2) (layer "F.Cu") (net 15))
 (segment (start 44.939108 177.95) (end 52.007108 170.882) (width 0.2) (layer "F.Cu") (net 15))
 (segment (start 28.240008 172.2) (end 27.240008 173.2) (width 0.2) (layer "F.Cu") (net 15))
 (segment (start 21.407108 173) (end 21.007108 173) (width 0.2) (layer "F.Cu") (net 15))
 (segment (start 46.507108 160.4) (end 24.707108 160.4) (width 0.2) (layer "F.Cu") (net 15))
 (segment (start 47.007108 160.9) (end 46.507108 160.4) (width 0.2) (layer "F.Cu") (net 15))
 (segment (start 52.007108 167) (end 52.007108 165.9) (width 0.2) (layer "F.Cu") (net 15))
 (segment (start 28.707108 172.2) (end 28.240008 172.2) (width 0.2) (layer "F.Cu") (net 15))
 (segment (start 24.707108 160.4) (end 21.407108 163.7) (width 0.2) (layer "F.Cu") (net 15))
 (segment (start 43.387108 177.95) (end 44.939108 177.95) (width 0.2) (layer "F.Cu") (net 15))
 (segment (start 21.407108 165) (end 21.407108 173) (width 0.2) (layer "F.Cu") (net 15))
 (segment (start 27.240008 173.2) (end 24.707108 173.2) (width 0.2) (layer "F.Cu") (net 15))
 (via (at 24.707108 173.2) (size 1) (drill 0.6) (layers "F.Cu" "B.Cu") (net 15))
 (via (at 21.007108 173) (size 1) (drill 0.6) (layers "F.Cu" "B.Cu") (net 15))
 (segment (start 21.207108 173.2) (end 21.007108 173) (width 0.2) (layer "B.Cu") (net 15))
 (segment (start 24.707108 173.2) (end 21.207108 173.2) (width 0.2) (layer "B.Cu") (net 15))
 (segment (start 36.114216 167.7) (end 30.707108 167.7) (width 0.2) (layer "F.Cu") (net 1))
 (segment (start 39.364216 170.95) (end 36.114216 167.7) (width 0.2) (layer "F.Cu") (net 1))
 (segment (start 26.707108 168.192893) (end 26.707108 168.2) (width 0.2) (layer "F.Cu") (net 1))
 (segment (start 30.207108 167.2) (end 27.700001 167.2) (width 0.2) (layer "F.Cu") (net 1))
 (segment (start 27.700001 167.2) (end 26.707108 168.192893) (width 0.2) (layer "F.Cu") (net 1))
 (segment (start 43.387108 170.95) (end 39.364216 170.95) (width 0.2) (layer "F.Cu") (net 1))
 (segment (start 30.707108 167.7) (end 30.207108 167.2) (width 0.2) (layer "F.Cu") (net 1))
 (segment (start 20.607108 170.8) (end 20.507108 170.9) (width 0.2) (layer "F.Cu") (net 16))
 (segment (start 27.140008 171.2) (end 24.707108 171.2) (width 0.2) (layer "F.Cu") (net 16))
 (segment (start 27.608108 170.799) (end 27.541008 170.799) (width 0.2) (layer "F.Cu") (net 16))
 (segment (start 20.807108 170.6) (end 20.607108 170.8) (width 0.2) (layer "F.Cu") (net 16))
 (segment (start 53.007108 167.1) (end 53.007108 165) (width 0.2) (layer "F.Cu") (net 16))
 (segment (start 28.707108 170.2) (end 28.207108 170.2) (width 0.2) (layer "F.Cu") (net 16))
 (segment (start 45.657108 178.45) (end 52.807108 171.3) (width 0.2) (layer "F.Cu") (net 16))
 (segment (start 28.207108 170.2) (end 27.608108 170.799) (width 0.2) (layer "F.Cu") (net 16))
 (segment (start 52.807108 171.3) (end 53.007108 171.1) (width 0.2) (layer "F.Cu") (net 16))
 (segment (start 43.387108 178.45) (end 45.657108 178.45) (width 0.2) (layer "F.Cu") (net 16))
 (segment (start 47.707108 159.7) (end 24.107108 159.7) (width 0.2) (layer "F.Cu") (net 16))
 (segment (start 20.807108 163) (end 20.807108 170.6) (width 0.2) (layer "F.Cu") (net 16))
 (segment (start 24.107108 159.7) (end 20.807108 163) (width 0.2) (layer "F.Cu") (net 16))
 (segment (start 53.007108 165) (end 47.707108 159.7) (width 0.2) (layer "F.Cu") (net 16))
 (segment (start 53.007108 171.1) (end 53.007108 167.1) (width 0.2) (layer "F.Cu") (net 16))
 (segment (start 27.541008 170.799) (end 27.140008 171.2) (width 0.2) (layer "F.Cu") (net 16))
 (via (at 24.707108 171.2) (size 1) (drill 0.6) (layers "F.Cu" "B.Cu") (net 16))
 (via (at 20.607108 170.8) (size 1) (drill 0.6) (layers "F.Cu" "B.Cu") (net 16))
 (segment (start 24.307108 170.8) (end 24.707108 171.2) (width 0.2) (layer "B.Cu") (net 16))
 (segment (start 20.607108 170.8) (end 24.307108 170.8) (width 0.2) (layer "B.Cu") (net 16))
 (segment (start 30.088423 179.581315) (end 29.707108 179.2) (width 0.2) (layer "F.Cu") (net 10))
 (segment (start 32.718685 179.581315) (end 30.088423 179.581315) (width 0.2) (layer "F.Cu") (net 10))
 (segment (start 43.387108 175.45) (end 36.85 175.45) (width 0.2) (layer "F.Cu") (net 10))
 (segment (start 36.85 175.45) (end 32.718685 179.581315) (width 0.2) (layer "F.Cu") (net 10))
 (segment (start 27.707108 179.2) (end 26.707108 180.2) (width 0.2) (layer "F.Cu") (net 10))
 (segment (start 29.707108 179.2) (end 27.707108 179.2) (width 0.2) (layer "F.Cu") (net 10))
 (segment (start 30.525793 176.581315) (end 29.907108 177.2) (width 0.2) (layer "F.Cu") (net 9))
 (segment (start 27.707108 177.2) (end 26.707108 178.2) (width 0.2) (layer "F.Cu") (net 9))
 (segment (start 43.387108 174.95) (end 35.664216 174.95) (width 0.2) (layer "F.Cu") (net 9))
 (segment (start 29.907108 177.2) (end 27.707108 177.2) (width 0.2) (layer "F.Cu") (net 9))
 (segment (start 34.032901 176.581315) (end 30.525793 176.581315) (width 0.2) (layer "F.Cu") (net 9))
 (segment (start 35.664216 174.95) (end 34.032901 176.581315) (width 0.2) (layer "F.Cu") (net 9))
 (segment (start 44.807108 162.8) (end 47.107108 165.1) (width 0.2) (layer "F.Cu") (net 5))
 (segment (start 27.541008 180.799) (end 27.140008 181.2) (width 0.2) (layer "F.Cu") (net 5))
 (segment (start 25.007108 181.2) (end 23.307108 179.5) (width 0.2) (layer "F.Cu") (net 5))
 (segment (start 28.707108 180.2) (end 28.207108 180.2) (width 0.2) (layer "F.Cu") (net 5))
 (segment (start 27.608108 180.799) (end 27.541008 180.799) (width 0.2) (layer "F.Cu") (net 5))
 (segment (start 47.107108 165.1) (end 47.107108 170.782) (width 0.2) (layer "F.Cu") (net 5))
 (segment (start 27.140008 181.2) (end 25.007108 181.2) (width 0.2) (layer "F.Cu") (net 5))
 (segment (start 25.007108 162.8) (end 44.807108 162.8) (width 0.2) (layer "F.Cu") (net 5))
 (segment (start 47.107108 170.782) (end 44.939108 172.95) (width 0.2) (layer "F.Cu") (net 5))
 (segment (start 28.207108 180.2) (end 27.608108 180.799) (width 0.2) (layer "F.Cu") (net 5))
 (segment (start 23.307108 164.5) (end 25.007108 162.8) (width 0.2) (layer "F.Cu") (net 5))
 (segment (start 44.939108 172.95) (end 43.387108 172.95) (width 0.2) (layer "F.Cu") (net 5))
 (segment (start 23.307108 179.5) (end 23.307108 164.5) (width 0.2) (layer "F.Cu") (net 5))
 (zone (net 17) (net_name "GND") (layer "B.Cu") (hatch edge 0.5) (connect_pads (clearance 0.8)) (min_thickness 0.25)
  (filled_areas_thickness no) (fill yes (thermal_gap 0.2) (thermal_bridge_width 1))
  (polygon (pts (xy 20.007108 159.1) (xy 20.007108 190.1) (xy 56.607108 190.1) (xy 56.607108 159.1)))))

